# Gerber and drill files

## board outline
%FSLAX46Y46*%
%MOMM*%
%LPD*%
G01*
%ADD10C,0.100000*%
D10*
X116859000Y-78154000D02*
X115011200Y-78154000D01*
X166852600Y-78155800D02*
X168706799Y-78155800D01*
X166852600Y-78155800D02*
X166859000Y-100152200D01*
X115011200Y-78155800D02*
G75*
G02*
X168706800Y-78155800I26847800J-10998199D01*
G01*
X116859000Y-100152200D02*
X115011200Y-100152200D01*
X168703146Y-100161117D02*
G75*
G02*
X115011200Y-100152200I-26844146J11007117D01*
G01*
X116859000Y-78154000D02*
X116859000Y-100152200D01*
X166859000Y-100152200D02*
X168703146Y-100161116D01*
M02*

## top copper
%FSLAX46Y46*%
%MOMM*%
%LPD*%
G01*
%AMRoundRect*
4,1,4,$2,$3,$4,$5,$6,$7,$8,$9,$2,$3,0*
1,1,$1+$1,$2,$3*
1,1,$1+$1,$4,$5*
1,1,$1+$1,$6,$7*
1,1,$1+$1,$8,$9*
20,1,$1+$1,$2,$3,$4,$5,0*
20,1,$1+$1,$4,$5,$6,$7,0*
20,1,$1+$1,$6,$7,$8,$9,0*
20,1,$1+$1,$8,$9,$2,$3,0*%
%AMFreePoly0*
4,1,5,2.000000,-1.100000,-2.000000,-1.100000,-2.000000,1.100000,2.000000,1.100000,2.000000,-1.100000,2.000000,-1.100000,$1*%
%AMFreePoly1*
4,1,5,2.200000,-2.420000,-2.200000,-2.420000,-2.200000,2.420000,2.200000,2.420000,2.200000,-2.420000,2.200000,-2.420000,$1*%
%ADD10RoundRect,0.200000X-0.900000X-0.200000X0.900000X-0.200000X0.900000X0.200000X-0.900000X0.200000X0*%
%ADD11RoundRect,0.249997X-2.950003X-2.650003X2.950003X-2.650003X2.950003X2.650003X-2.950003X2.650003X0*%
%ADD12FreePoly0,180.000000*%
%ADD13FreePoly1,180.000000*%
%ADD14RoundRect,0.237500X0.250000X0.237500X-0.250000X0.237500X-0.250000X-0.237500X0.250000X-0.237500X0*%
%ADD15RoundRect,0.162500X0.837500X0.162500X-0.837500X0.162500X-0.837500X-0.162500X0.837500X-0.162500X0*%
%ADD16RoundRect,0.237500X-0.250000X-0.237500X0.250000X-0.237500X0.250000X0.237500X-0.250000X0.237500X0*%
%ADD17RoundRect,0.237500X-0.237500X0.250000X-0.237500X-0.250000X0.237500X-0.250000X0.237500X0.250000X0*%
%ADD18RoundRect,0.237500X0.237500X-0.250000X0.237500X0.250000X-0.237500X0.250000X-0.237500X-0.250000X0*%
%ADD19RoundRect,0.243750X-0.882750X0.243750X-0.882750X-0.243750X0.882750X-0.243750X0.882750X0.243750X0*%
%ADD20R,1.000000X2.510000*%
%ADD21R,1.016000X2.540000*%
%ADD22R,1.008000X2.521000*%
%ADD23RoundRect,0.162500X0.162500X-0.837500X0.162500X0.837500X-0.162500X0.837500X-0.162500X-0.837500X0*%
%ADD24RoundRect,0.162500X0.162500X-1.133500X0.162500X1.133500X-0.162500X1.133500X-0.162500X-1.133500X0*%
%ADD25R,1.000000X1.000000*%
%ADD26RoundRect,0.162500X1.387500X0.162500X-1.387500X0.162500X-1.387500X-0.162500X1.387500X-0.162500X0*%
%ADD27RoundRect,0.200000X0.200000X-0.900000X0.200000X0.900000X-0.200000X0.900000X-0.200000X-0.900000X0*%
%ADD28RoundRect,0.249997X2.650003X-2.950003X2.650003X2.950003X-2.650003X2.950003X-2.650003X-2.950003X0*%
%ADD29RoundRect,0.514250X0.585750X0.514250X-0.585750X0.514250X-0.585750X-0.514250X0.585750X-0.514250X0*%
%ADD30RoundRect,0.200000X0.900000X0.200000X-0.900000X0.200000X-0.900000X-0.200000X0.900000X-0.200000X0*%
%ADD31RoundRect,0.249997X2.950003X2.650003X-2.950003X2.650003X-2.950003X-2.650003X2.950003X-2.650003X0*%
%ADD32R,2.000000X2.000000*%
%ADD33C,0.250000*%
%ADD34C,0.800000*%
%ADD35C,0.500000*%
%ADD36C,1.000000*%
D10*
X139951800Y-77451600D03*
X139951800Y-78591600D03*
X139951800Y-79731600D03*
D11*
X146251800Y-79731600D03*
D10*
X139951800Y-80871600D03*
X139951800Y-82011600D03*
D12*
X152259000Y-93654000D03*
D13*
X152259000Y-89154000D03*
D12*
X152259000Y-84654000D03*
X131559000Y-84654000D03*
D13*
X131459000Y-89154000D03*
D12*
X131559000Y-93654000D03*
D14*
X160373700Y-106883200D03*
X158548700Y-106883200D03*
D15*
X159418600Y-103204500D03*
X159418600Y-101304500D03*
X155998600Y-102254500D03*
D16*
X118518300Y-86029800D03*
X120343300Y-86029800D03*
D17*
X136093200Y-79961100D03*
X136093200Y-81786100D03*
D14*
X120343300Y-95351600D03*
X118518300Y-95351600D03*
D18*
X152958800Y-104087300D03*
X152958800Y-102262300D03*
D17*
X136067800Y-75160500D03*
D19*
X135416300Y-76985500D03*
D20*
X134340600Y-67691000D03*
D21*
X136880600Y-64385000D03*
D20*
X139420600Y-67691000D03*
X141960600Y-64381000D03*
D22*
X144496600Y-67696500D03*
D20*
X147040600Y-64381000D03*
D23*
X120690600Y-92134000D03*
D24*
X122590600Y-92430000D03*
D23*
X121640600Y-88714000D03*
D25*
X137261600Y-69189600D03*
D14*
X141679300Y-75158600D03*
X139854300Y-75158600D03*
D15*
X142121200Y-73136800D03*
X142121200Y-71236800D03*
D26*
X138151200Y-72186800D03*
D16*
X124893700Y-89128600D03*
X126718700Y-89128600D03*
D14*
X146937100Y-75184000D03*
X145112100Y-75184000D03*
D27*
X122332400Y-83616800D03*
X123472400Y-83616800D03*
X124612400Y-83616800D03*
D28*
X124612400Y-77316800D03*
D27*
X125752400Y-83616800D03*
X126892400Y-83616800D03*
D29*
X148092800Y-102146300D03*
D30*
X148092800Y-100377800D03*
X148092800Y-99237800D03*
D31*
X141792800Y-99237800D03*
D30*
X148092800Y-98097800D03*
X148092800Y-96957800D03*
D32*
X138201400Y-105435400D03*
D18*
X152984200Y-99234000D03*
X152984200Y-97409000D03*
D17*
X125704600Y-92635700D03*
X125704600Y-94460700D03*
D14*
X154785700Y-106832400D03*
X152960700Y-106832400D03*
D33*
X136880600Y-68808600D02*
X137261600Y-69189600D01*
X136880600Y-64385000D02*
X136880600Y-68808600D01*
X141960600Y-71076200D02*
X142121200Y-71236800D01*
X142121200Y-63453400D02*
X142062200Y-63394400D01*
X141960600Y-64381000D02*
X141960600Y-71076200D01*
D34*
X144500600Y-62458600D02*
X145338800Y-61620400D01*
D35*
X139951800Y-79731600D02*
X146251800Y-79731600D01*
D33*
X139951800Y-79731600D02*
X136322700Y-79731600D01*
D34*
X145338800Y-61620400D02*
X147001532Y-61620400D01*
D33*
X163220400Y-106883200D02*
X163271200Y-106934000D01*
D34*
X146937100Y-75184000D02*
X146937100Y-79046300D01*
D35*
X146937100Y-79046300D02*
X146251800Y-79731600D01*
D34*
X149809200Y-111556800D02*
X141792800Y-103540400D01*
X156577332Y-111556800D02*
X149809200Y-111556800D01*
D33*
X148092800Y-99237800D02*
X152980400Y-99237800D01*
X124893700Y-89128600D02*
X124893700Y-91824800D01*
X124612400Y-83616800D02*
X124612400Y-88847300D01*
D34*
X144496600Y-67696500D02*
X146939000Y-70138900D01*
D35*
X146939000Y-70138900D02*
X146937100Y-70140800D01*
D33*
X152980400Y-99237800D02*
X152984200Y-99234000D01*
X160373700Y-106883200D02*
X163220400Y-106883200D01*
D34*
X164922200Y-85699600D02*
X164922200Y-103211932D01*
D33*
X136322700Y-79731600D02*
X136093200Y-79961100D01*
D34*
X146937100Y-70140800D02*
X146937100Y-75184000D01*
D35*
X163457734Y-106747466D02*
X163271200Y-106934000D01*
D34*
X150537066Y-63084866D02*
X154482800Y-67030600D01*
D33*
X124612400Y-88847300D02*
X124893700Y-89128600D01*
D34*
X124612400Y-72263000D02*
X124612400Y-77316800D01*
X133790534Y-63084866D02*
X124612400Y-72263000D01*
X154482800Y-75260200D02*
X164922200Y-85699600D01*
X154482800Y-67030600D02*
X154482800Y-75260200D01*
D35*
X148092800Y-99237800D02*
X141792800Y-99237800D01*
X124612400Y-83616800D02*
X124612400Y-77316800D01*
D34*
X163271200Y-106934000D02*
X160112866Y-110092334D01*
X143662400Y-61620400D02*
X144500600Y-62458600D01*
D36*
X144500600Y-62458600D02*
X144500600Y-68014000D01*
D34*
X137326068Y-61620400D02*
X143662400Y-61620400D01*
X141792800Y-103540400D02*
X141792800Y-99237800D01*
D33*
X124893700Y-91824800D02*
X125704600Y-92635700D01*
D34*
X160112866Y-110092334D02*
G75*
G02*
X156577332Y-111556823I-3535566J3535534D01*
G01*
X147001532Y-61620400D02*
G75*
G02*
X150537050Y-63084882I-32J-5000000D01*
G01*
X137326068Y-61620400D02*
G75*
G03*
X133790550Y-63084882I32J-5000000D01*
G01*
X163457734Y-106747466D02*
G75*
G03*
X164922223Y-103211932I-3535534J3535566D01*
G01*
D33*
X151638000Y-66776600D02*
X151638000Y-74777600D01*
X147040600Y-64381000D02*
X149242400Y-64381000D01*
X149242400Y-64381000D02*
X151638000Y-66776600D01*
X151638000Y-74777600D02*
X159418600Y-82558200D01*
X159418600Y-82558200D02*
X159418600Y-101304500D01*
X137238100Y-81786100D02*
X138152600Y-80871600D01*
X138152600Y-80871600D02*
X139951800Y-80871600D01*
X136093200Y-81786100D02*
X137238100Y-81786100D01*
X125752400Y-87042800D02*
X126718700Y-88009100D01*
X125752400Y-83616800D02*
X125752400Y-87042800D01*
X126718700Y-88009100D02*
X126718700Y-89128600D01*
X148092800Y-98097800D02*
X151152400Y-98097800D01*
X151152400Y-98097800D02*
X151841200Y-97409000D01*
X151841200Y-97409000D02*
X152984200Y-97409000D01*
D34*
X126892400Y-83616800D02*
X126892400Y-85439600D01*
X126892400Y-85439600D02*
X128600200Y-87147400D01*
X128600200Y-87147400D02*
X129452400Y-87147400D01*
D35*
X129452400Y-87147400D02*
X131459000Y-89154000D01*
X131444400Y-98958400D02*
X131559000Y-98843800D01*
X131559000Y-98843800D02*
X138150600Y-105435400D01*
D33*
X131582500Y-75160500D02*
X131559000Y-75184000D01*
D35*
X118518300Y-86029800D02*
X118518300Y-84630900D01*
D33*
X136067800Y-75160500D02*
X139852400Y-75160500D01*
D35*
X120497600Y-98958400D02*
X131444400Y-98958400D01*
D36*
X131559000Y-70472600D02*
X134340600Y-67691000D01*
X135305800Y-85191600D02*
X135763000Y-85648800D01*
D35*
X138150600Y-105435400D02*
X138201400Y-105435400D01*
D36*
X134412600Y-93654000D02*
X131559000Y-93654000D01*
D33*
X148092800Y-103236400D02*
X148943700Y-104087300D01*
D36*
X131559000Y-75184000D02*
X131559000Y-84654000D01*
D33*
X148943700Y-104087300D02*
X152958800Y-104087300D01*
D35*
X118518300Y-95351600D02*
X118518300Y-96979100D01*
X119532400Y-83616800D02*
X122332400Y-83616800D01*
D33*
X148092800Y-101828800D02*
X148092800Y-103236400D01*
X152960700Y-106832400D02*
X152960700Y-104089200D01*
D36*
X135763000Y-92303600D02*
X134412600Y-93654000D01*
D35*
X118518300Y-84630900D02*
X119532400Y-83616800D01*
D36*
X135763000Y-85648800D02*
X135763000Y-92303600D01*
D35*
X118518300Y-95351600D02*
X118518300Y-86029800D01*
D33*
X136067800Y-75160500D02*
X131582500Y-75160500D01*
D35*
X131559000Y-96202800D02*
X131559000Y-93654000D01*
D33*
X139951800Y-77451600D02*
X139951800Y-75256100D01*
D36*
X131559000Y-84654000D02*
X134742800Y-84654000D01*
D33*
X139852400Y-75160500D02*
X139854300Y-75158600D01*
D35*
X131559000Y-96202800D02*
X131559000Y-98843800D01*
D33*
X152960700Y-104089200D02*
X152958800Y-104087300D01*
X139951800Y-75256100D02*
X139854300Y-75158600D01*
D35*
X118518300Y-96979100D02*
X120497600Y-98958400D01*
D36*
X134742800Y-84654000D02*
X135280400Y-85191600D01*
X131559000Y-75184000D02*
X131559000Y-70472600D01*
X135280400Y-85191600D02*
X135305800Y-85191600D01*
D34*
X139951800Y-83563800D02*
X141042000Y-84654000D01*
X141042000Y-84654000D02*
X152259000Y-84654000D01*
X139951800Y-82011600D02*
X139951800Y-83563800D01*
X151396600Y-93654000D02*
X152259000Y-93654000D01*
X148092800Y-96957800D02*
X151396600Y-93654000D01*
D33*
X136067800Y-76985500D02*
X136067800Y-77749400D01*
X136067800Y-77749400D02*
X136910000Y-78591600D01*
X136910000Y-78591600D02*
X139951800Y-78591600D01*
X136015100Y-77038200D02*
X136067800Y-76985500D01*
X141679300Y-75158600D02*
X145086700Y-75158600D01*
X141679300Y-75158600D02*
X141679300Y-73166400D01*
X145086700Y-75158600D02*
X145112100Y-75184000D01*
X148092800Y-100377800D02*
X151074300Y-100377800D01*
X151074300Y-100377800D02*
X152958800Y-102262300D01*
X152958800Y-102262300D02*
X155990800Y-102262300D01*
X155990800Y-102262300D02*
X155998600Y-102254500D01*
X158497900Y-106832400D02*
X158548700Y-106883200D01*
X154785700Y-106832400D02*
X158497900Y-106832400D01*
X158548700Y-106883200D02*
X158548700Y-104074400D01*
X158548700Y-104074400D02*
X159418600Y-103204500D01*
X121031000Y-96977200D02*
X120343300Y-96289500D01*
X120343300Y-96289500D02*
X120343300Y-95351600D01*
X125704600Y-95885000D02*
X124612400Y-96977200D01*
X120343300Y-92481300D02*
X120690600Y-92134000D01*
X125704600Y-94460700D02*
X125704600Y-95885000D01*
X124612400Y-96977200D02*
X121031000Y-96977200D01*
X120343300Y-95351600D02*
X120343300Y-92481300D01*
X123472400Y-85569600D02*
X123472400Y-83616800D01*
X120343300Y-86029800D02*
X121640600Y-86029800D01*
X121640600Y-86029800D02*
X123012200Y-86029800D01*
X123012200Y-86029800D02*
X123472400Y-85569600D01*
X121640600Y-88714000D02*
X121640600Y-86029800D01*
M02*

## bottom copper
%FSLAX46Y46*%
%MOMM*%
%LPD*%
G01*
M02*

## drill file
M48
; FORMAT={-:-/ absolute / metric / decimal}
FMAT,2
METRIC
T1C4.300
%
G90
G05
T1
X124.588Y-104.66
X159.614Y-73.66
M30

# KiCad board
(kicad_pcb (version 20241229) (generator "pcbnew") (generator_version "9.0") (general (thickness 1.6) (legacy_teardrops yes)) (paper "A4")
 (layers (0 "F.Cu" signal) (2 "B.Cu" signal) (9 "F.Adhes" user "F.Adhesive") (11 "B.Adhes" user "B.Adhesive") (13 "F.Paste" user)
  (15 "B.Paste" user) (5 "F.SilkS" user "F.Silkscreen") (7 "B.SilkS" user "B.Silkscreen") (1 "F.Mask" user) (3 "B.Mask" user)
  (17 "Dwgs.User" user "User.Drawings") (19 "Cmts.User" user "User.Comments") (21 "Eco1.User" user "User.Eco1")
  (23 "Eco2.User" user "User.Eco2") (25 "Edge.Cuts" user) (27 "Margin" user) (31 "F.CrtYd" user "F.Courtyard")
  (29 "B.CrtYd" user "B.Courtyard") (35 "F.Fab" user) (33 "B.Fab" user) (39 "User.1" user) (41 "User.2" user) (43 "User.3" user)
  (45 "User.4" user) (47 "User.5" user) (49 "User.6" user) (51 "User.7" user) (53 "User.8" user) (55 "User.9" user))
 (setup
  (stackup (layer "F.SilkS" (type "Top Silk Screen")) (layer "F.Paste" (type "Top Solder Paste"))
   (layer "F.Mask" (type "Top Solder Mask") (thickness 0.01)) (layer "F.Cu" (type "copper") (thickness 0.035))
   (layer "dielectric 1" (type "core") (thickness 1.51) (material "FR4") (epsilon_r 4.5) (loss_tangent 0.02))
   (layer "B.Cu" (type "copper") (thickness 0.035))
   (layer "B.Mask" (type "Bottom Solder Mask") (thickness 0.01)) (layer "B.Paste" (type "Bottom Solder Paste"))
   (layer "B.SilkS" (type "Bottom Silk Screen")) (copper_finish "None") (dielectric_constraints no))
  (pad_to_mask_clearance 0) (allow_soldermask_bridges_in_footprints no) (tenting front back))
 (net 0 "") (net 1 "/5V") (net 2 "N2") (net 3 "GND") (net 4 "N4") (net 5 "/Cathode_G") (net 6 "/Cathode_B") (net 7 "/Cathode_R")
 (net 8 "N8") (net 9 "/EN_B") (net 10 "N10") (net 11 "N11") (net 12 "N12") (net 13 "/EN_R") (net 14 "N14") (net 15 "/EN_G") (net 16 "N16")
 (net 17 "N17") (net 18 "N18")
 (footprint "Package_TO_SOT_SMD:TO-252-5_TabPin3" (layer "F.Cu") (at 144.9918 79.7316)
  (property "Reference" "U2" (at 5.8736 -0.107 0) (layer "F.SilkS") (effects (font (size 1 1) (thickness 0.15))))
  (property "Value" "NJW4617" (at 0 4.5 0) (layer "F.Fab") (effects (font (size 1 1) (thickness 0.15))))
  (pad "" smd roundrect (at -0.415 -1.525) (size 3.05 2.75) (layers "F.Paste") (roundrect_rratio 0.090909))
  (pad "" smd roundrect (at -0.415 1.525) (size 3.05 2.75) (layers "F.Paste") (roundrect_rratio 0.090909))
  (pad "" smd roundrect (at 2.935 -1.525) (size 3.05 2.75) (layers "F.Paste") (roundrect_rratio 0.090909))
  (pad "" smd roundrect (at 2.935 1.525) (size 3.05 2.75) (layers "F.Paste") (roundrect_rratio 0.090909))
  (pad "1" smd roundrect (at -5.04 -2.28) (size 2.2 0.8) (layers "F.Cu" "F.Mask" "F.Paste") (roundrect_rratio 0.25) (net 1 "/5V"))
  (pad "2" smd roundrect (at -5.04 -1.14) (size 2.2 0.8) (layers "F.Cu" "F.Mask" "F.Paste") (roundrect_rratio 0.25) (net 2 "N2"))
  (pad "3" smd roundrect (at -5.04 0) (size 2.2 0.8) (layers "F.Cu" "F.Mask" "F.Paste") (roundrect_rratio 0.25) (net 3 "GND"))
  (pad "3" smd roundrect (at 1.26 0) (size 6.4 5.8) (layers "F.Cu" "F.Mask") (roundrect_rratio 0.043103) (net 3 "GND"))
  (pad "4" smd roundrect (at -5.04 1.14) (size 2.2 0.8) (layers "F.Cu" "F.Mask" "F.Paste") (roundrect_rratio 0.25) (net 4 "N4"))
  (pad "5" smd roundrect (at -5.04 2.28) (size 2.2 0.8) (layers "F.Cu" "F.Mask" "F.Paste") (roundrect_rratio 0.25) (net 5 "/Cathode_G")))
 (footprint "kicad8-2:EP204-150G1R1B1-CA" (layer "F.Cu") (at 141.859 89.154 180)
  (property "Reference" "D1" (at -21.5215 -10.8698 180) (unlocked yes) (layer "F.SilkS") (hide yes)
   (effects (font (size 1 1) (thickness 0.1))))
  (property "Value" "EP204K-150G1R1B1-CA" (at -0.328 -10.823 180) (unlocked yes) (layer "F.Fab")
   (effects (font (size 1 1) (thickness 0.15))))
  (pad "1" smd custom (at -10.4 -4.5 180) (size 4 2.2) (layers "F.Cu" "F.Mask" "F.Paste") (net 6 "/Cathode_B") (thermal_bridge_angle 45)
   (options (clearance outline) (anchor rect)) (primitives))
  (pad "2" smd custom (at -10.4 0 180) (size 4.4 4.84) (layers "F.Cu" "F.Mask" "F.Paste") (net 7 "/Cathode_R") (thermal_bridge_angle 45)
   (options (clearance outline) (anchor rect)) (primitives))
  (pad "3" smd custom (at -10.4 4.5 180) (size 4 2.2) (layers "F.Cu" "F.Mask" "F.Paste") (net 5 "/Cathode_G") (thermal_bridge_angle 45)
   (options (clearance outline) (anchor rect)) (primitives))
  (pad "4" smd custom (at 10.3 4.5 180) (size 4 2.2) (layers "F.Cu" "F.Mask" "F.Paste") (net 1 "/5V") (thermal_bridge_angle 45)
   (options (clearance outline) (anchor rect)) (primitives))
  (pad "5" smd custom (at 10.4 0 180) (size 4.4 4.84) (layers "F.Cu" "F.Mask" "F.Paste") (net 7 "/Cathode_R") (thermal_bridge_angle 45)
   (options (clearance outline) (anchor rect)) (primitives))
  (pad "6" smd custom (at 10.3 -4.5 180) (size 4 2.2) (layers "F.Cu" "F.Mask" "F.Paste") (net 1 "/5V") (thermal_bridge_angle 45)
   (options (clearance outline) (anchor rect)) (primitives)))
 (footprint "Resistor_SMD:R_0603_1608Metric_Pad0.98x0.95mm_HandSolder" (layer "F.Cu") (at 159.4612 106.8832 180)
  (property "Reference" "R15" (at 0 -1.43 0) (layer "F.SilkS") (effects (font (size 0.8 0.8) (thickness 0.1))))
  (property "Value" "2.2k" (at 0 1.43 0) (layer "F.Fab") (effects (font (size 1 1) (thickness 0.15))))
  (pad "1" smd roundrect (at -0.9125 0 180) (size 0.975 0.95) (layers "F.Cu" "F.Mask" "F.Paste") (roundrect_rratio 0.25) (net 3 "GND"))
  (pad "2" smd roundrect (at 0.9125 0 180) (size 0.975 0.95) (layers "F.Cu" "F.Mask" "F.Paste") (roundrect_rratio 0.25) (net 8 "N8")))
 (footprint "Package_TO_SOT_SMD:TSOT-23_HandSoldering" (layer "F.Cu") (at 157.7086 102.2545 180)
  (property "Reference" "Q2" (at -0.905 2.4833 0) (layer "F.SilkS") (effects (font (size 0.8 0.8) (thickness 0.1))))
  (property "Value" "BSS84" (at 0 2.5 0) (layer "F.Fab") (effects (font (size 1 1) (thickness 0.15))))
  (pad "1" smd roundrect (at -1.71 -0.95 180) (size 2 0.65) (layers "F.Cu" "F.Mask" "F.Paste") (roundrect_rratio 0.25) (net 8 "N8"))
  (pad "2" smd roundrect (at -1.71 0.95 180) (size 2 0.65) (layers "F.Cu" "F.Mask" "F.Paste") (roundrect_rratio 0.25) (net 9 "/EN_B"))
  (pad "3" smd roundrect (at 1.71 0 180) (size 2 0.65) (layers "F.Cu" "F.Mask" "F.Paste") (roundrect_rratio 0.25) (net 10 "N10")))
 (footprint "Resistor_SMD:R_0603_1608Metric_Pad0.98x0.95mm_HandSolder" (layer "F.Cu") (at 119.4308 86.0298)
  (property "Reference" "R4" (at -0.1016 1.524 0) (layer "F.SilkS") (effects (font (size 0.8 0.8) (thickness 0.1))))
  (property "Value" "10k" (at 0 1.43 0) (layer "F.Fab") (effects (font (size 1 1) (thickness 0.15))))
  (pad "1" smd roundrect (at -0.9125 0) (size 0.975 0.95) (layers "F.Cu" "F.Mask" "F.Paste") (roundrect_rratio 0.25) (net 1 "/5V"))
  (pad "2" smd roundrect (at 0.9125 0) (size 0.975 0.95) (layers "F.Cu" "F.Mask" "F.Paste") (roundrect_rratio 0.25) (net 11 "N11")))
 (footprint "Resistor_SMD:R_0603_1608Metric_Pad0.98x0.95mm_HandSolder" (layer "F.Cu") (at 136.0932 80.8736 -90)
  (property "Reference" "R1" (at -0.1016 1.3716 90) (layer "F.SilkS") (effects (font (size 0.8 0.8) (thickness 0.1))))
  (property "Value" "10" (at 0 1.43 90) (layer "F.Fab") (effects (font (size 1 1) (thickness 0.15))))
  (pad "1" smd roundrect (at -0.9125 0 270) (size 0.975 0.95) (layers "F.Cu" "F.Mask" "F.Paste") (roundrect_rratio 0.25) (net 3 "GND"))
  (pad "2" smd roundrect (at 0.9125 0 270) (size 0.975 0.95) (layers "F.Cu" "F.Mask" "F.Paste") (roundrect_rratio 0.25) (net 4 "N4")))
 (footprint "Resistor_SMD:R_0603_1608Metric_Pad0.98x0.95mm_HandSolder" (layer "F.Cu") (at 119.4308 95.3516 180)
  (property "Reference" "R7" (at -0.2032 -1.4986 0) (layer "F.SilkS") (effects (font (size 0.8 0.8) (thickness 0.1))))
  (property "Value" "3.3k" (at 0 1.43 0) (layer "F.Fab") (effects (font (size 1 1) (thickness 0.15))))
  (pad "1" smd roundrect (at -0.9125 0 180) (size 0.975 0.95) (layers "F.Cu" "F.Mask" "F.Paste") (roundrect_rratio 0.25) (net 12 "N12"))
  (pad "2" smd roundrect (at 0.9125 0 180) (size 0.975 0.95) (layers "F.Cu" "F.Mask" "F.Paste") (roundrect_rratio 0.25) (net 1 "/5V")))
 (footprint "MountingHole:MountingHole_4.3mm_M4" (layer "F.Cu") (at 124.5882 104.66)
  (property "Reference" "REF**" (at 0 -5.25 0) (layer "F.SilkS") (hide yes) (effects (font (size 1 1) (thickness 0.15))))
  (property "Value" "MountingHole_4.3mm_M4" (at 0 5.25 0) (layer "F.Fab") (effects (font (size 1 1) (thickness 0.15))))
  (pad "" np_thru_hole circle (at 0 0) (size 4.3 4.3) (drill 4.3) (layers "*.Cu" "*.Mask")))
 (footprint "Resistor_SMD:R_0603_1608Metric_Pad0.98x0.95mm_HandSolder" (layer "F.Cu") (at 152.9588 103.1748 90)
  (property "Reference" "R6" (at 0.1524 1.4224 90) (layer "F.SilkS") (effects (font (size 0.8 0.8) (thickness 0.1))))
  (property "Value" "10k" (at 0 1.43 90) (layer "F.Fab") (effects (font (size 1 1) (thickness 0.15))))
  (pad "1" smd roundrect (at -0.9125 0 90) (size 0.975 0.95) (layers "F.Cu" "F.Mask" "F.Paste") (roundrect_rratio 0.25) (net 1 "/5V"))
  (pad "2" smd roundrect (at 0.9125 0 90) (size 0.975 0.95) (layers "F.Cu" "F.Mask" "F.Paste") (roundrect_rratio 0.25) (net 10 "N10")))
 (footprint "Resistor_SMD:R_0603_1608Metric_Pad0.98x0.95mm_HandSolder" (layer "F.Cu") (at 136.0678 76.073 -90)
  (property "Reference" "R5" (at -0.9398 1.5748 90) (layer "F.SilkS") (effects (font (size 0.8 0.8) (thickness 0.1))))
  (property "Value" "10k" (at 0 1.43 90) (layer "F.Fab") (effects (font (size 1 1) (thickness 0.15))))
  (pad "1" smd roundrect (at -0.9125 0 270) (size 0.975 0.95) (layers "F.Cu" "F.Mask" "F.Paste") (roundrect_rratio 0.25) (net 1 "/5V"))
  (pad "2" smd roundrect (at 0.9125 0.6515 270) (size 0.975 2.253) (layers "F.Cu" "F.Mask" "F.Paste") (roundrect_rratio 0.25) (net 2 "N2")))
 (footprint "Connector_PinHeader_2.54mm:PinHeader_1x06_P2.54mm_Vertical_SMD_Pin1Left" (layer "F.Cu") (at 140.6906 66.036 90)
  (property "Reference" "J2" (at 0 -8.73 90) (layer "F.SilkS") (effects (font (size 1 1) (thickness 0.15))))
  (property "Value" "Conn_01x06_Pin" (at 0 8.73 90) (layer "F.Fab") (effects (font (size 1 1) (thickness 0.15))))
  (pad "1" smd rect (at -1.655 -6.35 90) (size 2.51 1) (layers "F.Cu" "F.Mask" "F.Paste") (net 1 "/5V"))
  (pad "2" smd rect (at 1.651 -3.81 90) (size 2.54 1.016) (layers "F.Cu" "F.Mask" "F.Paste") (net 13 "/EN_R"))
  (pad "3" smd rect (at -1.655 -1.27 90) (size 2.51 1) (layers "F.Cu" "F.Mask" "F.Paste") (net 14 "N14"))
  (pad "4" smd rect (at 1.655 1.27 90) (size 2.51 1) (layers "F.Cu" "F.Mask" "F.Paste") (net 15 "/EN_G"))
  (pad "5" smd rect (at -1.6605 3.806 90) (size 2.521 1.008) (layers "F.Cu" "F.Mask" "F.Paste") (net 3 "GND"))
  (pad "6" smd rect (at 1.655 6.35 90) (size 2.51 1) (layers "F.Cu" "F.Mask" "F.Paste") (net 9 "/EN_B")))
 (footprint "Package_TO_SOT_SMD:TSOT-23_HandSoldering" (layer "F.Cu") (at 121.6406 90.424 90)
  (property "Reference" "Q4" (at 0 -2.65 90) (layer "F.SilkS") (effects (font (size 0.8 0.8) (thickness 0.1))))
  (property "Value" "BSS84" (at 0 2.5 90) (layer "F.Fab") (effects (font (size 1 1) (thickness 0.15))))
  (pad "1" smd roundrect (at -1.71 -0.95 90) (size 2 0.65) (layers "F.Cu" "F.Mask" "F.Paste") (roundrect_rratio 0.25) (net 12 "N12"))
  (pad "2" smd roundrect (at -2.006 0.95 90) (size 2.592 0.65) (layers "F.Cu" "F.Mask" "F.Paste") (roundrect_rratio 0.25) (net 13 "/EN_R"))
  (pad "3" smd roundrect (at 1.71 0 90) (size 2 0.65) (layers "F.Cu" "F.Mask" "F.Paste") (roundrect_rratio 0.25) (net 11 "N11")))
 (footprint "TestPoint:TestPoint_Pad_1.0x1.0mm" (layer "F.Cu") (at 137.2616 69.1896)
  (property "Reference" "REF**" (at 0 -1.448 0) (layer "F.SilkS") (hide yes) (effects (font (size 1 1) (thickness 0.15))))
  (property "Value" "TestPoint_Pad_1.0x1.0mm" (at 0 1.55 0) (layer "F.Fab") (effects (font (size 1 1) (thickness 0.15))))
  (pad "1" smd rect (at 0 0) (size 1 1) (layers "F.Cu" "F.Mask") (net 13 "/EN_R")))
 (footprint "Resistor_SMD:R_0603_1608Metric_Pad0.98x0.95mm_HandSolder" (layer "F.Cu") (at 140.7668 75.1586 180)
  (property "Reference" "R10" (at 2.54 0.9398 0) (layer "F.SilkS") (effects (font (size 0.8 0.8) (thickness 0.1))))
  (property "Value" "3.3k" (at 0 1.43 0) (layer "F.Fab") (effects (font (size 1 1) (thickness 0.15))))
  (pad "1" smd roundrect (at -0.9125 0 180) (size 0.975 0.95) (layers "F.Cu" "F.Mask" "F.Paste") (roundrect_rratio 0.25) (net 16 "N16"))
  (pad "2" smd roundrect (at 0.9125 0 180) (size 0.975 0.95) (layers "F.Cu" "F.Mask" "F.Paste") (roundrect_rratio 0.25) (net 1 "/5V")))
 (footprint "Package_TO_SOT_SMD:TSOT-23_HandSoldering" (layer "F.Cu") (at 140.4112 72.1868 180)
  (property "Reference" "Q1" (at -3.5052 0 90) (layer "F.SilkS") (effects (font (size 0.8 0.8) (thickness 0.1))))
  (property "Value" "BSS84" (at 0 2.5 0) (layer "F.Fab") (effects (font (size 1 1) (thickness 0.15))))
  (pad "1" smd roundrect (at -1.71 -0.95 180) (size 2 0.65) (layers "F.Cu" "F.Mask" "F.Paste") (roundrect_rratio 0.25) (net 16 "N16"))
  (pad "2" smd roundrect (at -1.71 0.95 180) (size 2 0.65) (layers "F.Cu" "F.Mask" "F.Paste") (roundrect_rratio 0.25) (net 15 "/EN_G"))
  (pad "3" smd roundrect (at 2.26 0 180) (size 3.1 0.65) (layers "F.Cu" "F.Mask" "F.Paste") (roundrect_rratio 0.25) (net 2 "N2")))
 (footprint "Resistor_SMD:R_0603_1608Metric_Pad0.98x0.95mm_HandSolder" (layer "F.Cu") (at 125.8062 89.1286)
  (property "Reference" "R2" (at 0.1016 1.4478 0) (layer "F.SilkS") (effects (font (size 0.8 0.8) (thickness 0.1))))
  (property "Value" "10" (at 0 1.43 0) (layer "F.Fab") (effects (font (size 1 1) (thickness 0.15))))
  (pad "1" smd roundrect (at -0.9125 0) (size 0.975 0.95) (layers "F.Cu" "F.Mask" "F.Paste") (roundrect_rratio 0.25) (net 3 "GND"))
  (pad "2" smd roundrect (at 0.9125 0) (size 0.975 0.95) (layers "F.Cu" "F.Mask" "F.Paste") (roundrect_rratio 0.25) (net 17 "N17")))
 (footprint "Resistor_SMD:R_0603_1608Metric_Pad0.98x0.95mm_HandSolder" (layer "F.Cu") (at 146.0246 75.184 180)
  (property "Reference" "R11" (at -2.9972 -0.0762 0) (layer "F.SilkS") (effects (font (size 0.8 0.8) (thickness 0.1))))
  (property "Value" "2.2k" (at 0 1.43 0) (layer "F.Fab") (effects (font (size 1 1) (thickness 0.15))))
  (pad "1" smd roundrect (at -0.9125 0 180) (size 0.975 0.95) (layers "F.Cu" "F.Mask" "F.Paste") (roundrect_rratio 0.25) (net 3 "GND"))
  (pad "2" smd roundrect (at 0.9125 0 180) (size 0.975 0.95) (layers "F.Cu" "F.Mask" "F.Paste") (roundrect_rratio 0.25) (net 16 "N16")))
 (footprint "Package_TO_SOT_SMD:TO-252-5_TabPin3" (layer "F.Cu") (at 124.6124 78.5768 90)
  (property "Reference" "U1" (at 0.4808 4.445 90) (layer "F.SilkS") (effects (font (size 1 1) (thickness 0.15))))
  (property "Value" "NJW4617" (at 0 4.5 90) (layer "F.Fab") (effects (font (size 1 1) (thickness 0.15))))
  (pad "" smd roundrect (at -0.415 -1.525 90) (size 3.05 2.75) (layers "F.Paste") (roundrect_rratio 0.090909))
  (pad "" smd roundrect (at -0.415 1.525 90) (size 3.05 2.75) (layers "F.Paste") (roundrect_rratio 0.090909))
  (pad "" smd roundrect (at 2.935 -1.525 90) (size 3.05 2.75) (layers "F.Paste") (roundrect_rratio 0.090909))
  (pad "" smd roundrect (at 2.935 1.525 90) (size 3.05 2.75) (layers "F.Paste") (roundrect_rratio 0.090909))
  (pad "1" smd roundrect (at -5.04 -2.28 90) (size 2.2 0.8) (layers "F.Cu" "F.Mask" "F.Paste") (roundrect_rratio 0.25) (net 1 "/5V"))
  (pad "2" smd roundrect (at -5.04 -1.14 90) (size 2.2 0.8) (layers "F.Cu" "F.Mask" "F.Paste") (roundrect_rratio 0.25) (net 11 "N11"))
  (pad "3" smd roundrect (at -5.04 0 90) (size 2.2 0.8) (layers "F.Cu" "F.Mask" "F.Paste") (roundrect_rratio 0.25) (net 3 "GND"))
  (pad "3" smd roundrect (at 1.26 0 90) (size 6.4 5.8) (layers "F.Cu" "F.Mask") (roundrect_rratio 0.043103) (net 3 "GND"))
  (pad "4" smd roundrect (at -5.04 1.14 90) (size 2.2 0.8) (layers "F.Cu" "F.Mask" "F.Paste") (roundrect_rratio 0.25) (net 17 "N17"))
  (pad "5" smd roundrect (at -5.04 2.28 90) (size 2.2 0.8) (layers "F.Cu" "F.Mask" "F.Paste") (roundrect_rratio 0.25) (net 7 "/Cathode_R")))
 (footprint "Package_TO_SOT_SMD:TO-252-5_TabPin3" (layer "F.Cu") (at 143.0528 99.2378 180)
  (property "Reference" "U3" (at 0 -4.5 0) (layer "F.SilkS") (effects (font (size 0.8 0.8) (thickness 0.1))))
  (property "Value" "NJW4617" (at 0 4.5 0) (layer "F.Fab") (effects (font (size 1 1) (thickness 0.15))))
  (pad "" smd roundrect (at -0.415 -1.525 180) (size 3.05 2.75) (layers "F.Paste") (roundrect_rratio 0.090909))
  (pad "" smd roundrect (at -0.415 1.525 180) (size 3.05 2.75) (layers "F.Paste") (roundrect_rratio 0.090909))
  (pad "" smd roundrect (at 2.935 -1.525 180) (size 3.05 2.75) (layers "F.Paste") (roundrect_rratio 0.090909))
  (pad "" smd roundrect (at 2.935 1.525 180) (size 3.05 2.75) (layers "F.Paste") (roundrect_rratio 0.090909))
  (pad "1" smd roundrect (at -5.04 -2.9085 180) (size 2.2 2.057) (layers "F.Cu" "F.Mask" "F.Paste") (roundrect_rratio 0.25) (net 1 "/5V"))
  (pad "2" smd roundrect (at -5.04 -1.14 180) (size 2.2 0.8) (layers "F.Cu" "F.Mask" "F.Paste") (roundrect_rratio 0.25) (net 10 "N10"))
  (pad "3" smd roundrect (at -5.04 0 180) (size 2.2 0.8) (layers "F.Cu" "F.Mask" "F.Paste") (roundrect_rratio 0.25) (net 3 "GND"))
  (pad "3" smd roundrect (at 1.26 0 180) (size 6.4 5.8) (layers "F.Cu" "F.Mask") (roundrect_rratio 0.043103) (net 3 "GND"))
  (pad "4" smd roundrect (at -5.04 1.14 180) (size 2.2 0.8) (layers "F.Cu" "F.Mask" "F.Paste") (roundrect_rratio 0.25) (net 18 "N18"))
  (pad "5" smd roundrect (at -5.04 2.28 180) (size 2.2 0.8) (layers "F.Cu" "F.Mask" "F.Paste") (roundrect_rratio 0.25) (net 6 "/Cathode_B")))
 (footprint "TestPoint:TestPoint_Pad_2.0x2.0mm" (layer "F.Cu") (at 138.2014 105.4354)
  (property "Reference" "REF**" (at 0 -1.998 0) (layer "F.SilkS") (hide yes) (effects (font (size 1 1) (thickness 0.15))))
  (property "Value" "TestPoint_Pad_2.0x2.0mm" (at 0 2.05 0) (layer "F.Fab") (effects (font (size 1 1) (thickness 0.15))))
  (pad "1" smd rect (at 0 0) (size 2 2) (layers "F.Cu" "F.Mask") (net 1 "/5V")))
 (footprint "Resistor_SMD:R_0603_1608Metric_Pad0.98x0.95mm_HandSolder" (layer "F.Cu") (at 152.9842 98.3215 90)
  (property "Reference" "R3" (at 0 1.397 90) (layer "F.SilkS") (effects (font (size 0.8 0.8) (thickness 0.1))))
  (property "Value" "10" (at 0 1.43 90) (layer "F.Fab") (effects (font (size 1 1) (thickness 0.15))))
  (pad "1" smd roundrect (at -0.9125 0 90) (size 0.975 0.95) (layers "F.Cu" "F.Mask" "F.Paste") (roundrect_rratio 0.25) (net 3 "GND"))
  (pad "2" smd roundrect (at 0.9125 0 90) (size 0.975 0.95) (layers "F.Cu" "F.Mask" "F.Paste") (roundrect_rratio 0.25) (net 18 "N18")))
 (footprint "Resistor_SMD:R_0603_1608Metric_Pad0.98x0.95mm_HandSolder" (layer "F.Cu") (at 125.7046 93.5482 -90)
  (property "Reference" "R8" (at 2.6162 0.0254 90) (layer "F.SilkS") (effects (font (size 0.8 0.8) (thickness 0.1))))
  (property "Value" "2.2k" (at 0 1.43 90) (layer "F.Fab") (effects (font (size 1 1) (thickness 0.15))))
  (pad "1" smd roundrect (at -0.9125 0 270) (size 0.975 0.95) (layers "F.Cu" "F.Mask" "F.Paste") (roundrect_rratio 0.25) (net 3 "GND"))
  (pad "2" smd roundrect (at 0.9125 0 270) (size 0.975 0.95) (layers "F.Cu" "F.Mask" "F.Paste") (roundrect_rratio 0.25) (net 12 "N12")))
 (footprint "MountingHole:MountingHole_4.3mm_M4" (layer "F.Cu") (at 159.6136 73.66)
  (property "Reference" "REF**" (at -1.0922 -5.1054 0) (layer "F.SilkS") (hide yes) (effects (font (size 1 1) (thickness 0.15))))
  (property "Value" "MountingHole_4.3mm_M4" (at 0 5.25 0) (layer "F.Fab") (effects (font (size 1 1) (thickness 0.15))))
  (pad "" np_thru_hole circle (at 0 0) (size 4.3 4.3) (drill 4.3) (layers "*.Cu" "*.Mask")))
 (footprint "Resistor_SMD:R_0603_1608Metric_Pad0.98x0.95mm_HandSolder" (layer "F.Cu") (at 153.8732 106.8324 180)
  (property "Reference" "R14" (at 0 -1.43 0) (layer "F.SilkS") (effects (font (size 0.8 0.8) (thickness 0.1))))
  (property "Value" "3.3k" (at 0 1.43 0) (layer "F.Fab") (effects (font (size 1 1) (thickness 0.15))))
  (pad "1" smd roundrect (at -0.9125 0 180) (size 0.975 0.95) (layers "F.Cu" "F.Mask" "F.Paste") (roundrect_rratio 0.25) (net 8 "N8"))
  (pad "2" smd roundrect (at 0.9125 0 180) (size 0.975 0.95) (layers "F.Cu" "F.Mask" "F.Paste") (roundrect_rratio 0.25) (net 1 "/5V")))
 (gr_line (start 116.859 78.154) (end 115.0112 78.154) (stroke (width 0.1) (type default)) (layer "Edge.Cuts"))
 (gr_line (start 166.8526 78.1558) (end 168.706799 78.1558) (stroke (width 0.1) (type default)) (layer "Edge.Cuts"))
 (gr_line (start 166.8526 78.1558) (end 166.859 100.1522) (stroke (width 0.1) (type default)) (layer "Edge.Cuts"))
 (gr_arc (start 115.0112 78.1558) (mid 141.859 60.140817) (end 168.7068 78.1558) (stroke (width 0.1) (type default)) (layer "Edge.Cuts"))
 (gr_line (start 116.859 100.1522) (end 115.0112 100.1522) (stroke (width 0.1) (type default)) (layer "Edge.Cuts"))
 (gr_arc (start 168.703146 100.161117) (mid 141.854182 118.167183) (end 115.0112 100.1522) (stroke (width 0.1) (type default))
  (layer "Edge.Cuts"))
 (gr_line (start 116.859 78.154) (end 116.859 100.1522) (stroke (width 0.1) (type default)) (layer "Edge.Cuts"))
 (gr_line (start 166.859 100.1522) (end 168.703146 100.161116) (stroke (width 0.1) (type default)) (layer "Edge.Cuts"))
 (segment (start 136.8806 68.8086) (end 137.2616 69.1896) (width 0.25) (layer "F.Cu") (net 13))
 (segment (start 136.8806 64.385) (end 136.8806 68.8086) (width 0.25) (layer "F.Cu") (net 13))
 (segment (start 141.9606 71.0762) (end 142.1212 71.2368) (width 0.25) (layer "F.Cu") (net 15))
 (segment (start 142.1212 63.4534) (end 142.0622 63.3944) (width 0.25) (layer "F.Cu") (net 15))
 (segment (start 141.9606 64.381) (end 141.9606 71.0762) (width 0.25) (layer "F.Cu") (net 15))
 (segment (start 144.5006 62.4586) (end 145.3388 61.6204) (width 0.8) (layer "F.Cu") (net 3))
 (segment (start 139.9518 79.7316) (end 146.2518 79.7316) (width 0.5) (layer "F.Cu") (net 3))
 (segment (start 139.9518 79.7316) (end 136.3227 79.7316) (width 0.25) (layer "F.Cu") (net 3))
 (segment (start 145.3388 61.6204) (end 147.001532 61.6204) (width 0.8) (layer "F.Cu") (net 3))
 (segment (start 163.2204 106.8832) (end 163.2712 106.934) (width 0.25) (layer "F.Cu") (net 3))
 (segment (start 146.9371 75.184) (end 146.9371 79.0463) (width 0.8) (layer "F.Cu") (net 3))
 (segment (start 146.9371 79.0463) (end 146.2518 79.7316) (width 0.5) (layer "F.Cu") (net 3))
 (segment (start 149.8092 111.5568) (end 141.7928 103.5404) (width 0.8) (layer "F.Cu") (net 3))
 (segment (start 156.577332 111.5568) (end 149.8092 111.5568) (width 0.8) (layer "F.Cu") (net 3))
 (segment (start 148.0928 99.2378) (end 152.9804 99.2378) (width 0.25) (layer "F.Cu") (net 3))
 (segment (start 124.8937 89.1286) (end 124.8937 91.8248) (width 0.25) (layer "F.Cu") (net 3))
 (segment (start 124.6124 83.6168) (end 124.6124 88.8473) (width 0.25) (layer "F.Cu") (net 3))
 (segment (start 144.4966 67.6965) (end 146.939 70.1389) (width 0.8) (layer "F.Cu") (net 3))
 (segment (start 146.939 70.1389) (end 146.9371 70.1408) (width 0.5) (layer "F.Cu") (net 3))
 (segment (start 152.9804 99.2378) (end 152.9842 99.234) (width 0.25) (layer "F.Cu") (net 3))
 (segment (start 160.3737 106.8832) (end 163.2204 106.8832) (width 0.25) (layer "F.Cu") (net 3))
 (segment (start 164.9222 85.6996) (end 164.9222 103.211932) (width 0.8) (layer "F.Cu") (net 3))
 (segment (start 136.3227 79.7316) (end 136.0932 79.9611) (width 0.25) (layer "F.Cu") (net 3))
 (segment (start 146.9371 70.1408) (end 146.9371 75.184) (width 0.8) (layer "F.Cu") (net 3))
 (segment (start 163.457734 106.747466) (end 163.2712 106.934) (width 0.5) (layer "F.Cu") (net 3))
 (segment (start 150.537066 63.084866) (end 154.4828 67.0306) (width 0.8) (layer "F.Cu") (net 3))
 (segment (start 124.6124 88.8473) (end 124.8937 89.1286) (width 0.25) (layer "F.Cu") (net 3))
 (segment (start 124.6124 72.263) (end 124.6124 77.3168) (width 0.8) (layer "F.Cu") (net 3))
 (segment (start 133.790534 63.084866) (end 124.6124 72.263) (width 0.8) (layer "F.Cu") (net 3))
 (segment (start 154.4828 75.2602) (end 164.9222 85.6996) (width 0.8) (layer "F.Cu") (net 3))
 (segment (start 154.4828 67.0306) (end 154.4828 75.2602) (width 0.8) (layer "F.Cu") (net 3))
 (segment (start 148.0928 99.2378) (end 141.7928 99.2378) (width 0.5) (layer "F.Cu") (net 3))
 (segment (start 124.6124 83.6168) (end 124.6124 77.3168) (width 0.5) (layer "F.Cu") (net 3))
 (segment (start 163.2712 106.934) (end 160.112866 110.092334) (width 0.8) (layer "F.Cu") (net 3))
 (segment (start 143.6624 61.6204) (end 144.5006 62.4586) (width 0.8) (layer "F.Cu") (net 3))
 (segment (start 144.5006 62.4586) (end 144.5006 68.014) (width 1) (layer "F.Cu") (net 3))
 (segment (start 137.326068 61.6204) (end 143.6624 61.6204) (width 0.8) (layer "F.Cu") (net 3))
 (segment (start 141.7928 103.5404) (end 141.7928 99.2378) (width 0.8) (layer "F.Cu") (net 3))
 (segment (start 124.8937 91.8248) (end 125.7046 92.6357) (width 0.25) (layer "F.Cu") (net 3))
 (arc (start 160.112866 110.092334) (mid 158.490749 111.176198) (end 156.577332 111.5568) (width 0.8) (layer "F.Cu") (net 3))
 (arc (start 147.001532 61.6204) (mid 148.914949 62.001002) (end 150.537066 63.084866) (width 0.8) (layer "F.Cu") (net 3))
 (arc (start 137.326068 61.6204) (mid 135.412651 62.001002) (end 133.790534 63.084866) (width 0.8) (layer "F.Cu") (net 3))
 (arc (start 163.457734 106.747466) (mid 164.541598 105.125349) (end 164.9222 103.211932) (width 0.8) (layer "F.Cu") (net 3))
 (segment (start 151.638 66.7766) (end 151.638 74.7776) (width 0.25) (layer "F.Cu") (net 9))
 (segment (start 147.0406 64.381) (end 149.2424 64.381) (width 0.25) (layer "F.Cu") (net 9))
 (segment (start 149.2424 64.381) (end 151.638 66.7766) (width 0.25) (layer "F.Cu") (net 9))
 (segment (start 151.638 74.7776) (end 159.4186 82.5582) (width 0.25) (layer "F.Cu") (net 9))
 (segment (start 159.4186 82.5582) (end 159.4186 101.3045) (width 0.25) (layer "F.Cu") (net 9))
 (segment (start 137.2381 81.7861) (end 138.1526 80.8716) (width 0.25) (layer "F.Cu") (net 4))
 (segment (start 138.1526 80.8716) (end 139.9518 80.8716) (width 0.25) (layer "F.Cu") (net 4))
 (segment (start 136.0932 81.7861) (end 137.2381 81.7861) (width 0.25) (layer "F.Cu") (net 4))
 (segment (start 125.7524 87.0428) (end 126.7187 88.0091) (width 0.25) (layer "F.Cu") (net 17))
 (segment (start 125.7524 83.6168) (end 125.7524 87.0428) (width 0.25) (layer "F.Cu") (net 17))
 (segment (start 126.7187 88.0091) (end 126.7187 89.1286) (width 0.25) (layer "F.Cu") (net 17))
 (segment (start 148.0928 98.0978) (end 151.1524 98.0978) (width 0.25) (layer "F.Cu") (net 18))
 (segment (start 151.1524 98.0978) (end 151.8412 97.409) (width 0.25) (layer "F.Cu") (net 18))
 (segment (start 151.8412 97.409) (end 152.9842 97.409) (width 0.25) (layer "F.Cu") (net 18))
 (segment (start 126.8924 83.6168) (end 126.8924 85.4396) (width 0.8) (layer "F.Cu") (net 7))
 (segment (start 126.8924 85.4396) (end 128.6002 87.1474) (width 0.8) (layer "F.Cu") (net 7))
 (segment (start 128.6002 87.1474) (end 129.4524 87.1474) (width 0.8) (layer "F.Cu") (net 7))
 (segment (start 129.4524 87.1474) (end 131.459 89.154) (width 0.5) (layer "F.Cu") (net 7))
 (segment (start 131.4444 98.9584) (end 131.559 98.8438) (width 0.5) (layer "F.Cu") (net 1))
 (segment (start 131.559 98.8438) (end 138.1506 105.4354) (width 0.5) (layer "F.Cu") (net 1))
 (segment (start 131.5825 75.1605) (end 131.559 75.184) (width 0.25) (layer "F.Cu") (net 1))
 (segment (start 118.5183 86.0298) (end 118.5183 84.6309) (width 0.5) (layer "F.Cu") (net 1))
 (segment (start 136.0678 75.1605) (end 139.8524 75.1605) (width 0.25) (layer "F.Cu") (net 1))
 (segment (start 120.4976 98.9584) (end 131.4444 98.9584) (width 0.5) (layer "F.Cu") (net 1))
 (segment (start 131.559 70.4726) (end 134.3406 67.691) (width 1) (layer "F.Cu") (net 1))
 (segment (start 135.3058 85.1916) (end 135.763 85.6488) (width 1) (layer "F.Cu") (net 1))
 (segment (start 138.1506 105.4354) (end 138.2014 105.4354) (width 0.5) (layer "F.Cu") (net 1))
 (segment (start 134.4126 93.654) (end 131.559 93.654) (width 1) (layer "F.Cu") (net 1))
 (segment (start 148.0928 103.2364) (end 148.9437 104.0873) (width 0.25) (layer "F.Cu") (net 1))
 (segment (start 131.559 75.184) (end 131.559 84.654) (width 1) (layer "F.Cu") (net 1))
 (segment (start 148.9437 104.0873) (end 152.9588 104.0873) (width 0.25) (layer "F.Cu") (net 1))
 (segment (start 118.5183 95.3516) (end 118.5183 96.9791) (width 0.5) (layer "F.Cu") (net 1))
 (segment (start 119.5324 83.6168) (end 122.3324 83.6168) (width 0.5) (layer "F.Cu") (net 1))
 (segment (start 148.0928 101.8288) (end 148.0928 103.2364) (width 0.25) (layer "F.Cu") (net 1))
 (segment (start 152.9607 106.8324) (end 152.9607 104.0892) (width 0.25) (layer "F.Cu") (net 1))
 (segment (start 135.763 92.3036) (end 134.4126 93.654) (width 1) (layer "F.Cu") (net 1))
 (segment (start 118.5183 84.6309) (end 119.5324 83.6168) (width 0.5) (layer "F.Cu") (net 1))
 (segment (start 135.763 85.6488) (end 135.763 92.3036) (width 1) (layer "F.Cu") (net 1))
 (segment (start 118.5183 95.3516) (end 118.5183 86.0298) (width 0.5) (layer "F.Cu") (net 1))
 (segment (start 136.0678 75.1605) (end 131.5825 75.1605) (width 0.25) (layer "F.Cu") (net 1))
 (segment (start 131.559 96.2028) (end 131.559 93.654) (width 0.5) (layer "F.Cu") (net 1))
 (segment (start 139.9518 77.4516) (end 139.9518 75.2561) (width 0.25) (layer "F.Cu") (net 1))
 (segment (start 131.559 84.654) (end 134.7428 84.654) (width 1) (layer "F.Cu") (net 1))
 (segment (start 139.8524 75.1605) (end 139.8543 75.1586) (width 0.25) (layer "F.Cu") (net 1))
 (segment (start 131.559 96.2028) (end 131.559 98.8438) (width 0.5) (layer "F.Cu") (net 1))
 (segment (start 152.9607 104.0892) (end 152.9588 104.0873) (width 0.25) (layer "F.Cu") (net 1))
 (segment (start 139.9518 75.2561) (end 139.8543 75.1586) (width 0.25) (layer "F.Cu") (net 1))
 (segment (start 118.5183 96.9791) (end 120.4976 98.9584) (width 0.5) (layer "F.Cu") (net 1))
 (segment (start 134.7428 84.654) (end 135.2804 85.1916) (width 1) (layer "F.Cu") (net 1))
 (segment (start 131.559 75.184) (end 131.559 70.4726) (width 1) (layer "F.Cu") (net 1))
 (segment (start 135.2804 85.1916) (end 135.3058 85.1916) (width 1) (layer "F.Cu") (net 1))
 (segment (start 139.9518 83.5638) (end 141.042 84.654) (width 0.8) (layer "F.Cu") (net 5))
 (segment (start 141.042 84.654) (end 152.259 84.654) (width 0.8) (layer "F.Cu") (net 5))
 (segment (start 139.9518 82.0116) (end 139.9518 83.5638) (width 0.8) (layer "F.Cu") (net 5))
 (segment (start 151.3966 93.654) (end 152.259 93.654) (width 0.8) (layer "F.Cu") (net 6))
 (segment (start 148.0928 96.9578) (end 151.3966 93.654) (width 0.8) (layer "F.Cu") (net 6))
 (segment (start 136.0678 76.9855) (end 136.0678 77.7494) (width 0.25) (layer "F.Cu") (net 2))
 (segment (start 136.0678 77.7494) (end 136.91 78.5916) (width 0.25) (layer "F.Cu") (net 2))
 (segment (start 136.91 78.5916) (end 139.9518 78.5916) (width 0.25) (layer "F.Cu") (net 2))
 (segment (start 136.0151 77.0382) (end 136.0678 76.9855) (width 0.25) (layer "F.Cu") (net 2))
 (segment (start 141.6793 75.1586) (end 145.0867 75.1586) (width 0.25) (layer "F.Cu") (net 16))
 (segment (start 141.6793 75.1586) (end 141.6793 73.1664) (width 0.25) (layer "F.Cu") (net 16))
 (segment (start 145.0867 75.1586) (end 145.1121 75.184) (width 0.25) (layer "F.Cu") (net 16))
 (segment (start 148.0928 100.3778) (end 151.0743 100.3778) (width 0.25) (layer "F.Cu") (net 10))
 (segment (start 151.0743 100.3778) (end 152.9588 102.2623) (width 0.25) (layer "F.Cu") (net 10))
 (segment (start 152.9588 102.2623) (end 155.9908 102.2623) (width 0.25) (layer "F.Cu") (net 10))
 (segment (start 155.9908 102.2623) (end 155.9986 102.2545) (width 0.25) (layer "F.Cu") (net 10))
 (segment (start 158.4979 106.8324) (end 158.5487 106.8832) (width 0.25) (layer "F.Cu") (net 8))
 (segment (start 154.7857 106.8324) (end 158.4979 106.8324) (width 0.25) (layer "F.Cu") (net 8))
 (segment (start 158.5487 106.8832) (end 158.5487 104.0744) (width 0.25) (layer "F.Cu") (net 8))
 (segment (start 158.5487 104.0744) (end 159.4186 103.2045) (width 0.25) (layer "F.Cu") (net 8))
 (segment (start 121.031 96.9772) (end 120.3433 96.2895) (width 0.25) (layer "F.Cu") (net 12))
 (segment (start 120.3433 96.2895) (end 120.3433 95.3516) (width 0.25) (layer "F.Cu") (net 12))
 (segment (start 125.7046 95.885) (end 124.6124 96.9772) (width 0.25) (layer "F.Cu") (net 12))
 (segment (start 120.3433 92.4813) (end 120.6906 92.134) (width 0.25) (layer "F.Cu") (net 12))
 (segment (start 125.7046 94.4607) (end 125.7046 95.885) (width 0.25) (layer "F.Cu") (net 12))
 (segment (start 124.6124 96.9772) (end 121.031 96.9772) (width 0.25) (layer "F.Cu") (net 12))
 (segment (start 120.3433 95.3516) (end 120.3433 92.4813) (width 0.25) (layer "F.Cu") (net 12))
 (segment (start 123.4724 85.5696) (end 123.4724 83.6168) (width 0.25) (layer "F.Cu") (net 11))
 (segment (start 120.3433 86.0298) (end 121.6406 86.0298) (width 0.25) (layer "F.Cu") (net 11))
 (segment (start 121.6406 86.0298) (end 123.0122 86.0298) (width 0.25) (layer "F.Cu") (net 11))
 (segment (start 123.0122 86.0298) (end 123.4724 85.5696) (width 0.25) (layer "F.Cu") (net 11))
 (segment (start 121.6406 88.714) (end 121.6406 86.0298) (width 0.25) (layer "F.Cu") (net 11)))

